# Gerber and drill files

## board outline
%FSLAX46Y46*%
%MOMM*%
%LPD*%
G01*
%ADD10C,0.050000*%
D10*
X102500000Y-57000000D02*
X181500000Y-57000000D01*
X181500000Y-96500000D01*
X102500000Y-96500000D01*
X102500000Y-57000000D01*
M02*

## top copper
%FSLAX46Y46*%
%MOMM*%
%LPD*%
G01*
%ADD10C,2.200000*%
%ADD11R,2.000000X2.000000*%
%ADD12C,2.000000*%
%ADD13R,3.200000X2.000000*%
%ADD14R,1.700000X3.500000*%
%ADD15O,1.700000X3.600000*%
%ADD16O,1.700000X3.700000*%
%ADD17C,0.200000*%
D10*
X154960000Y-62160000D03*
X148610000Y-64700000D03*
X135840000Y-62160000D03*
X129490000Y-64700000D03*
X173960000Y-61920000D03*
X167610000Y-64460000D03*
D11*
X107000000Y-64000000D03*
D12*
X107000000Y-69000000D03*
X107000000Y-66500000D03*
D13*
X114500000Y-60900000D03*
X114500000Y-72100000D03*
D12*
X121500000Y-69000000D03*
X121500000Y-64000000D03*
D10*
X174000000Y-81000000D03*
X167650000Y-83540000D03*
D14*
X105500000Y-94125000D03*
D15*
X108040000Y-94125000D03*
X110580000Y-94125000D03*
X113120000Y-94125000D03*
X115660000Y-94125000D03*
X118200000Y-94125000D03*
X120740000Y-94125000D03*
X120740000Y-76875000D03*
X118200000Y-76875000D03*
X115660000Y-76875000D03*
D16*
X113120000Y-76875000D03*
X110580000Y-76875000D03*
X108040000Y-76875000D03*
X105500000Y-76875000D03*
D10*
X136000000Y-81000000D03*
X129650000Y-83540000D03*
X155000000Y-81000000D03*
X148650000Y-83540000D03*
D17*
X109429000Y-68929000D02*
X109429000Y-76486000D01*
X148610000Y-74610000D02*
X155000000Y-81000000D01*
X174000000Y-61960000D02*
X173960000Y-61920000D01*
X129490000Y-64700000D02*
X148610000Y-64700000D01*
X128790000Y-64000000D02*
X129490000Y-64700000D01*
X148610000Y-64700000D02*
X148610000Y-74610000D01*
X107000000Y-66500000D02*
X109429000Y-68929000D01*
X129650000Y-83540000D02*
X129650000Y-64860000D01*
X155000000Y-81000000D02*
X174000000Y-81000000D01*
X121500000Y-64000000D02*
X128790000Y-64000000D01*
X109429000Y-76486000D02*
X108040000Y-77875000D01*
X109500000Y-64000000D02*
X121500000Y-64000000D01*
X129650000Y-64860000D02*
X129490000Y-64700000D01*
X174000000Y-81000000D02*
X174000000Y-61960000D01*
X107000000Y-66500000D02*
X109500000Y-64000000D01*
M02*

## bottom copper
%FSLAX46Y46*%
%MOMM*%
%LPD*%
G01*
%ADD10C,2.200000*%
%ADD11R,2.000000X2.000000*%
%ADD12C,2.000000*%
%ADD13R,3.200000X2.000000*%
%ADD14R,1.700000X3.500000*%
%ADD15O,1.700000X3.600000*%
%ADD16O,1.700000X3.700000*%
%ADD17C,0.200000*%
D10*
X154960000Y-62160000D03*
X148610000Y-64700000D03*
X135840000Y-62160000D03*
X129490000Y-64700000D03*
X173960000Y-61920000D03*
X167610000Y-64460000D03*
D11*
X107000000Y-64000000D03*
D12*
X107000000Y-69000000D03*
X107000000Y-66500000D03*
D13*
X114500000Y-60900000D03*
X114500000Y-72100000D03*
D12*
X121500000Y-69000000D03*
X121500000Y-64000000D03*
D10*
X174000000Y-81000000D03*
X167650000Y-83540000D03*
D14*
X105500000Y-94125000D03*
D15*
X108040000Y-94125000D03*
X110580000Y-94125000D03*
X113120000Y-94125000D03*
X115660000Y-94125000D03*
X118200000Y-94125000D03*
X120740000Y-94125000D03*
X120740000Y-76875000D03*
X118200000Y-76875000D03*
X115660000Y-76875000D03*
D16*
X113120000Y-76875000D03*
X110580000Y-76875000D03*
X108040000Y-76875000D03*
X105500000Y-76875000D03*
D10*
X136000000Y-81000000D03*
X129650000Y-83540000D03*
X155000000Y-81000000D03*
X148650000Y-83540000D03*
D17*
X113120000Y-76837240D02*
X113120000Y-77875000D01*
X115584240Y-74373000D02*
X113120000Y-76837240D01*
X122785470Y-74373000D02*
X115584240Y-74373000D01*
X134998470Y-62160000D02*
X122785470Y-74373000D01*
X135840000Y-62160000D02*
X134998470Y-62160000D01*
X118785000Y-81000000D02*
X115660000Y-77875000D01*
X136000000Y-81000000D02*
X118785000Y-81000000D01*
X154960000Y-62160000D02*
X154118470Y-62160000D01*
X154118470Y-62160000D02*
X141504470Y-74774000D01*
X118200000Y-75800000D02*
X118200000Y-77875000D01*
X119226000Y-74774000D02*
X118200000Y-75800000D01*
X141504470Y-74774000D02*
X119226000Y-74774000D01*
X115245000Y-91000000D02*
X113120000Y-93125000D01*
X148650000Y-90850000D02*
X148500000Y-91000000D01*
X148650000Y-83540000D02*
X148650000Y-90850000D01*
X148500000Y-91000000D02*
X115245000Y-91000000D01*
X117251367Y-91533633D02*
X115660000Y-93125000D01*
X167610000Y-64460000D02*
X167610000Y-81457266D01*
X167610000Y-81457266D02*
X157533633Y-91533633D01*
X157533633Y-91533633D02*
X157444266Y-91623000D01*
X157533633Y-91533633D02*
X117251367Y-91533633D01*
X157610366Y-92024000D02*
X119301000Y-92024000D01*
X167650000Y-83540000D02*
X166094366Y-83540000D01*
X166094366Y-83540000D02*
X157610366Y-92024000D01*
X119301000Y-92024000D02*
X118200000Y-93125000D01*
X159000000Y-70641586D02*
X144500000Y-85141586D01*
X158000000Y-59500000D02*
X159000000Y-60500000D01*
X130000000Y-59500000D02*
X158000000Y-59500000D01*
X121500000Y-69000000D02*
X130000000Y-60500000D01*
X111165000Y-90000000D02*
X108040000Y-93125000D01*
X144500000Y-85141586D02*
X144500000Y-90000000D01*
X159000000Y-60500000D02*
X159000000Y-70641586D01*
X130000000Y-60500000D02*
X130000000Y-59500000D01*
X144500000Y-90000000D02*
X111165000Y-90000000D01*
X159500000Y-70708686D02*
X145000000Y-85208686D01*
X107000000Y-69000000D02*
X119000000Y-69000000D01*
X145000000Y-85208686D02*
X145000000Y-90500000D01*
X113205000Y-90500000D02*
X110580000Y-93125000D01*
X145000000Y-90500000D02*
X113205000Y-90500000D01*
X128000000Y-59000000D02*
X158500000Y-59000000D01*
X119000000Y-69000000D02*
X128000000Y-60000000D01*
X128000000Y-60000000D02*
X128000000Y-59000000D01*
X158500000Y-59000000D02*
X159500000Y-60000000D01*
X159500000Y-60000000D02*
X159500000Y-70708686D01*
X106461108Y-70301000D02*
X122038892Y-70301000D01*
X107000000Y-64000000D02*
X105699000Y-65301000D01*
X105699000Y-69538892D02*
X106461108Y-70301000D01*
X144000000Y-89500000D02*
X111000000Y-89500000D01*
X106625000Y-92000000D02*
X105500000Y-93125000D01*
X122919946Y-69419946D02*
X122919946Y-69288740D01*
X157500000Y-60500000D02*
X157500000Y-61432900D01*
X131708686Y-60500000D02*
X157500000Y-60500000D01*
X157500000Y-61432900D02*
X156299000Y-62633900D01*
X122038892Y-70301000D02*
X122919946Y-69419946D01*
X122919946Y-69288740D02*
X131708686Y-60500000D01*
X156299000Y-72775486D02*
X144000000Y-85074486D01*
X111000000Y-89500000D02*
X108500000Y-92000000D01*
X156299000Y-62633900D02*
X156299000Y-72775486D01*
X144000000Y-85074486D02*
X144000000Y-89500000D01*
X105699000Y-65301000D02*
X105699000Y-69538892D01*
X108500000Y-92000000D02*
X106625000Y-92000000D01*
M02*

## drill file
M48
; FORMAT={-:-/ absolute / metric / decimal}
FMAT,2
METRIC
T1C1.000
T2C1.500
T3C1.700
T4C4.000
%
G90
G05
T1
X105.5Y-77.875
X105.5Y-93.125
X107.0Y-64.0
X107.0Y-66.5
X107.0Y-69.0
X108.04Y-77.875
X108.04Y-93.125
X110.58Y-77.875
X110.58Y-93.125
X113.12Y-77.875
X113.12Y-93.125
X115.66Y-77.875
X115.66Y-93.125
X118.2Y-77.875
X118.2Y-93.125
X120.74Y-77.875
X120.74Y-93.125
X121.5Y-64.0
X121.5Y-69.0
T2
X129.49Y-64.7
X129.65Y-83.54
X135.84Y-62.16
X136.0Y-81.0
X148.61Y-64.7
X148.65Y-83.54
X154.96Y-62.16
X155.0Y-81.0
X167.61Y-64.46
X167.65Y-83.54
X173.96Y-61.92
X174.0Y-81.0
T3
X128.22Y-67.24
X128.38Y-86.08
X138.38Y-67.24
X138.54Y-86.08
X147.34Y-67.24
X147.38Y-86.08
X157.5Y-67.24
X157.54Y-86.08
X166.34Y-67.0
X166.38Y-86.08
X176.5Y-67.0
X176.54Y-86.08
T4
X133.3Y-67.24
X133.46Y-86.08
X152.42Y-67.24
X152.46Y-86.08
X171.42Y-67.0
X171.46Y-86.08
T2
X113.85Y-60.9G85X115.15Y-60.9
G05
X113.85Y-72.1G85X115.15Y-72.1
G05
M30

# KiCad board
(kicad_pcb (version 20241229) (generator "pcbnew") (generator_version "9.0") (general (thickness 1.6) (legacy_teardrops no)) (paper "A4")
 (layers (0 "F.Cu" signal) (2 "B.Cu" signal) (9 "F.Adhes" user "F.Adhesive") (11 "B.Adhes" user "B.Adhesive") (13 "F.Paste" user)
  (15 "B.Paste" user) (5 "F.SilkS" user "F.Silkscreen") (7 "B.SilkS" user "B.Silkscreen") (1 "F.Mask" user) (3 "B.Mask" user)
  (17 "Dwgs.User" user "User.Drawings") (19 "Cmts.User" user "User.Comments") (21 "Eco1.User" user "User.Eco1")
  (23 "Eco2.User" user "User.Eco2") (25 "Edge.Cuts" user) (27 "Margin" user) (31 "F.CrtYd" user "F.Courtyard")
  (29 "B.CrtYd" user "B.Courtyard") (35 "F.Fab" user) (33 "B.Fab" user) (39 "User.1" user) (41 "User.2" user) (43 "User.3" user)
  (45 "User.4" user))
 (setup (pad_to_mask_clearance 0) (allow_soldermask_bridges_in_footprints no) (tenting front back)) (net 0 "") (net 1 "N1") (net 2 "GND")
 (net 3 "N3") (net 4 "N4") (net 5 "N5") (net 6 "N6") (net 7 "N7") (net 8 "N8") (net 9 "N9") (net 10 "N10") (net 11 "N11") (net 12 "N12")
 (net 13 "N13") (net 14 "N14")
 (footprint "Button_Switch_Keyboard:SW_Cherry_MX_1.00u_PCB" (layer "F.Cu") (at 154.96 62.16)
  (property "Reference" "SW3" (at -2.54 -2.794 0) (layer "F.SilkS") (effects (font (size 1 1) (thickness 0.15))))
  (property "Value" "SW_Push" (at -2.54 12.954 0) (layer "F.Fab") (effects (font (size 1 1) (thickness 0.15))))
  (pad "" np_thru_hole circle (at -7.62 5.08) (size 1.7 1.7) (drill 1.7) (layers "*.Cu" "*.Mask"))
  (pad "" np_thru_hole circle (at -2.54 5.08) (size 4 4) (drill 4) (layers "*.Cu" "*.Mask"))
  (pad "" np_thru_hole circle (at 2.54 5.08) (size 1.7 1.7) (drill 1.7) (layers "*.Cu" "*.Mask"))
  (pad "1" thru_hole circle (at 0 0) (size 2.2 2.2) (drill 1.5) (layers "*.Cu" "*.Mask") (remove_unused_layers no) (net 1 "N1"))
  (pad "2" thru_hole circle (at -6.35 2.54) (size 2.2 2.2) (drill 1.5) (layers "*.Cu" "*.Mask") (remove_unused_layers no) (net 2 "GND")))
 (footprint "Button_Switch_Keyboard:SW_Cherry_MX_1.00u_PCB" (layer "F.Cu") (at 135.84 62.16)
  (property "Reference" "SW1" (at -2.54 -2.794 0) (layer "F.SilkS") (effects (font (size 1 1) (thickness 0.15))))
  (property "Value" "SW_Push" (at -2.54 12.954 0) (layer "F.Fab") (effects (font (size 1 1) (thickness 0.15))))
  (pad "" np_thru_hole circle (at -7.62 5.08) (size 1.7 1.7) (drill 1.7) (layers "*.Cu" "*.Mask"))
  (pad "" np_thru_hole circle (at -2.54 5.08) (size 4 4) (drill 4) (layers "*.Cu" "*.Mask"))
  (pad "" np_thru_hole circle (at 2.54 5.08) (size 1.7 1.7) (drill 1.7) (layers "*.Cu" "*.Mask"))
  (pad "1" thru_hole circle (at 0 0) (size 2.2 2.2) (drill 1.5) (layers "*.Cu" "*.Mask") (remove_unused_layers no) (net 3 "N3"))
  (pad "2" thru_hole circle (at -6.35 2.54) (size 2.2 2.2) (drill 1.5) (layers "*.Cu" "*.Mask") (remove_unused_layers no) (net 2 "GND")))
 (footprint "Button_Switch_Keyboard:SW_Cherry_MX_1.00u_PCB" (layer "F.Cu") (at 173.96 61.92)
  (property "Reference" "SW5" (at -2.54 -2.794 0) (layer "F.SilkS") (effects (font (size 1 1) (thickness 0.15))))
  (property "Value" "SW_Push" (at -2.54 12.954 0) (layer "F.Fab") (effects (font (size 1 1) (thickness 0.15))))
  (pad "" np_thru_hole circle (at -7.62 5.08) (size 1.7 1.7) (drill 1.7) (layers "*.Cu" "*.Mask"))
  (pad "" np_thru_hole circle (at -2.54 5.08) (size 4 4) (drill 4) (layers "*.Cu" "*.Mask"))
  (pad "" np_thru_hole circle (at 2.54 5.08) (size 1.7 1.7) (drill 1.7) (layers "*.Cu" "*.Mask"))
  (pad "1" thru_hole circle (at 0 0) (size 2.2 2.2) (drill 1.5) (layers "*.Cu" "*.Mask") (remove_unused_layers no) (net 2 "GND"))
  (pad "2" thru_hole circle (at -6.35 2.54) (size 2.2 2.2) (drill 1.5) (layers "*.Cu" "*.Mask") (remove_unused_layers no) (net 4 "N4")))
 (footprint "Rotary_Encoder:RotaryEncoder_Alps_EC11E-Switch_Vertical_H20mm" (layer "F.Cu") (at 107 64)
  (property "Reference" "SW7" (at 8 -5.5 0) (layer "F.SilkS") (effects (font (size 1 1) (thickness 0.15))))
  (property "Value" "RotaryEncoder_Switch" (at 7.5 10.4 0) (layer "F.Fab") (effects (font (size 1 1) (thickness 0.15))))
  (pad "A" thru_hole rect (at 0 0) (size 2 2) (drill 1) (layers "*.Cu" "*.Mask") (remove_unused_layers no) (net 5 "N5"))
  (pad "B" thru_hole circle (at 0 5) (size 2 2) (drill 1) (layers "*.Cu" "*.Mask") (remove_unused_layers no) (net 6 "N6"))
  (pad "C" thru_hole circle (at 0 2.5) (size 2 2) (drill 1) (layers "*.Cu" "*.Mask") (remove_unused_layers no) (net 2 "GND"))
  (pad "MP" thru_hole rect (at 7.5 -3.1) (size 3.2 2) (drill oval 2.8 1.5) (layers "*.Cu" "*.Mask") (remove_unused_layers no))
  (pad "MP" thru_hole rect (at 7.5 8.1) (size 3.2 2) (drill oval 2.8 1.5) (layers "*.Cu" "*.Mask") (remove_unused_layers no))
  (pad "S1" thru_hole circle (at 14.5 5) (size 2 2) (drill 1) (layers "*.Cu" "*.Mask") (remove_unused_layers no) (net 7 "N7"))
  (pad "S2" thru_hole circle (at 14.5 0) (size 2 2) (drill 1) (layers "*.Cu" "*.Mask") (remove_unused_layers no) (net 2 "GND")))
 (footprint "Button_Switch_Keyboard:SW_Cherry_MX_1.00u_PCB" (layer "F.Cu") (at 174 81)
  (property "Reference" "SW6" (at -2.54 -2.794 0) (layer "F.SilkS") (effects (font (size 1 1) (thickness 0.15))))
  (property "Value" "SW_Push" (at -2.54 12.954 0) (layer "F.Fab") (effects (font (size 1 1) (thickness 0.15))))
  (pad "" np_thru_hole circle (at -7.62 5.08) (size 1.7 1.7) (drill 1.7) (layers "*.Cu" "*.Mask"))
  (pad "" np_thru_hole circle (at -2.54 5.08) (size 4 4) (drill 4) (layers "*.Cu" "*.Mask"))
  (pad "" np_thru_hole circle (at 2.54 5.08) (size 1.7 1.7) (drill 1.7) (layers "*.Cu" "*.Mask"))
  (pad "1" thru_hole circle (at 0 0) (size 2.2 2.2) (drill 1.5) (layers "*.Cu" "*.Mask") (remove_unused_layers no) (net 2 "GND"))
  (pad "2" thru_hole circle (at -6.35 2.54) (size 2.2 2.2) (drill 1.5) (layers "*.Cu" "*.Mask") (remove_unused_layers no) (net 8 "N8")))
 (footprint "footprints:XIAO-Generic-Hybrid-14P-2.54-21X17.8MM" (layer "F.Cu") (at 113.12 85.5 90)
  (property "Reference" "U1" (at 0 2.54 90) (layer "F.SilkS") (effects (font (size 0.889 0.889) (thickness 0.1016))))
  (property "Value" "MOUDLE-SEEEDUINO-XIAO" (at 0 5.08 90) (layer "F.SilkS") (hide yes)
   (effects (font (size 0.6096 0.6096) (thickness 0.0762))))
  (pad "1" thru_hole rect (at -7.625 -7.62 90) (size 3.5 1.7) (drill 1 (offset -1 0)) (layers "*.Cu" "*.Mask") (remove_unused_layers no)
   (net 5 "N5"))
  (pad "2" thru_hole oval (at -7.625 -5.08 90) (size 3.6 1.7) (drill 1 (offset -1 0)) (layers "*.Cu" "*.Mask") (remove_unused_layers no)
   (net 7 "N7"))
  (pad "3" thru_hole oval (at -7.625 -2.54 90) (size 3.6 1.7) (drill 1 (offset -1 0)) (layers "*.Cu" "*.Mask") (remove_unused_layers no)
   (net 6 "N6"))
  (pad "4" thru_hole oval (at -7.625 0 90) (size 3.6 1.7) (drill 1 (offset -1 0)) (layers "*.Cu" "*.Mask") (remove_unused_layers no)
   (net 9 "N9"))
  (pad "5" thru_hole oval (at -7.625 2.54 90) (size 3.6 1.7) (drill 1 (offset -1 0)) (layers "*.Cu" "*.Mask") (remove_unused_layers no)
   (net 4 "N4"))
  (pad "6" thru_hole oval (at -7.625 5.08 270) (size 3.6 1.7) (drill 1 (offset 1 0)) (layers "*.Cu" "*.Mask") (remove_unused_layers no)
   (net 8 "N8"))
  (pad "7" thru_hole oval (at -7.625 7.62 90) (size 3.6 1.7) (drill 1 (offset -1 0)) (layers "*.Cu" "*.Mask") (remove_unused_layers no)
   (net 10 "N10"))
  (pad "8" thru_hole oval (at 7.625 7.62 90) (size 3.6 1.7) (drill 1 (offset 1 0)) (layers "*.Cu" "*.Mask") (remove_unused_layers no)
   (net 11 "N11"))
  (pad "9" thru_hole oval (at 7.625 5.08 90) (size 3.6 1.7) (drill 1 (offset 1 0)) (layers "*.Cu" "*.Mask") (remove_unused_layers no)
   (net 1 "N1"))
  (pad "10" thru_hole oval (at 7.625 2.54 90) (size 3.6 1.7) (drill 1 (offset 1 0)) (layers "*.Cu" "*.Mask") (remove_unused_layers no)
   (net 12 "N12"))
  (pad "11" thru_hole oval (at 7.625 0 90) (size 3.7 1.7) (drill 1 (offset 1 0)) (layers "*.Cu" "*.Mask") (remove_unused_layers no)
   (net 3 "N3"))
  (pad "12" thru_hole oval (at 7.625 -2.54 90) (size 3.7 1.7) (drill 1 (offset 1 0)) (layers "*.Cu" "*.Mask") (remove_unused_layers no)
   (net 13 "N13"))
  (pad "13" thru_hole oval (at 7.625 -5.08 90) (size 3.7 1.7) (drill 1 (offset 1 0)) (layers "*.Cu" "*.Mask") (remove_unused_layers no)
   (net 2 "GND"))
  (pad "14" thru_hole oval (at 7.625 -7.62 90) (size 3.7 1.7) (drill 1 (offset 1 0)) (layers "*.Cu" "*.Mask") (remove_unused_layers no)
   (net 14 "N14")))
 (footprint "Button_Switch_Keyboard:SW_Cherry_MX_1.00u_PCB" (layer "F.Cu") (at 136 81)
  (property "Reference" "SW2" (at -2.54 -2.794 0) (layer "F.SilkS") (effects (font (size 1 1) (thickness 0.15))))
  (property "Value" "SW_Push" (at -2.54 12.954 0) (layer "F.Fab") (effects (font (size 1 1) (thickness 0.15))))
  (pad "" np_thru_hole circle (at -7.62 5.08) (size 1.7 1.7) (drill 1.7) (layers "*.Cu" "*.Mask"))
  (pad "" np_thru_hole circle (at -2.54 5.08) (size 4 4) (drill 4) (layers "*.Cu" "*.Mask"))
  (pad "" np_thru_hole circle (at 2.54 5.08) (size 1.7 1.7) (drill 1.7) (layers "*.Cu" "*.Mask"))
  (pad "1" thru_hole circle (at 0 0) (size 2.2 2.2) (drill 1.5) (layers "*.Cu" "*.Mask") (remove_unused_layers no) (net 12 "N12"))
  (pad "2" thru_hole circle (at -6.35 2.54) (size 2.2 2.2) (drill 1.5) (layers "*.Cu" "*.Mask") (remove_unused_layers no) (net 2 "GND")))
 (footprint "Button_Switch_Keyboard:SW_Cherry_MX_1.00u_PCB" (layer "F.Cu") (at 155 81)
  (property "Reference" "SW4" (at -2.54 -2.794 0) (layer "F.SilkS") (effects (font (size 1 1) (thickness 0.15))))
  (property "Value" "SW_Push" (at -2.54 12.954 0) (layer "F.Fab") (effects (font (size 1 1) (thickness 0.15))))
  (pad "" np_thru_hole circle (at -7.62 5.08) (size 1.7 1.7) (drill 1.7) (layers "*.Cu" "*.Mask"))
  (pad "" np_thru_hole circle (at -2.54 5.08) (size 4 4) (drill 4) (layers "*.Cu" "*.Mask"))
  (pad "" np_thru_hole circle (at 2.54 5.08) (size 1.7 1.7) (drill 1.7) (layers "*.Cu" "*.Mask"))
  (pad "1" thru_hole circle (at 0 0) (size 2.2 2.2) (drill 1.5) (layers "*.Cu" "*.Mask") (remove_unused_layers no) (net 2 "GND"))
  (pad "2" thru_hole circle (at -6.35 2.54) (size 2.2 2.2) (drill 1.5) (layers "*.Cu" "*.Mask") (remove_unused_layers no) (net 9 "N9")))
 (gr_rect (start 102.5 57) (end 181.5 96.5) (stroke (width 0.05) (type default)) (fill no) (layer "Edge.Cuts"))
 (segment (start 113.12 76.83724) (end 113.12 77.875) (width 0.2) (layer "B.Cu") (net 3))
 (segment (start 115.58424 74.373) (end 113.12 76.83724) (width 0.2) (layer "B.Cu") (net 3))
 (segment (start 122.78547 74.373) (end 115.58424 74.373) (width 0.2) (layer "B.Cu") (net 3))
 (segment (start 134.99847 62.16) (end 122.78547 74.373) (width 0.2) (layer "B.Cu") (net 3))
 (segment (start 135.84 62.16) (end 134.99847 62.16) (width 0.2) (layer "B.Cu") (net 3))
 (segment (start 109.429 68.929) (end 109.429 76.486) (width 0.2) (layer "F.Cu") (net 2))
 (segment (start 148.61 74.61) (end 155 81) (width 0.2) (layer "F.Cu") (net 2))
 (segment (start 174 61.96) (end 173.96 61.92) (width 0.2) (layer "F.Cu") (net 2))
 (segment (start 129.49 64.7) (end 148.61 64.7) (width 0.2) (layer "F.Cu") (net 2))
 (segment (start 128.79 64) (end 129.49 64.7) (width 0.2) (layer "F.Cu") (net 2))
 (segment (start 148.61 64.7) (end 148.61 74.61) (width 0.2) (layer "F.Cu") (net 2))
 (segment (start 107 66.5) (end 109.429 68.929) (width 0.2) (layer "F.Cu") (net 2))
 (segment (start 129.65 83.54) (end 129.65 64.86) (width 0.2) (layer "F.Cu") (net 2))
 (segment (start 155 81) (end 174 81) (width 0.2) (layer "F.Cu") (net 2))
 (segment (start 121.5 64) (end 128.79 64) (width 0.2) (layer "F.Cu") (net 2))
 (segment (start 109.429 76.486) (end 108.04 77.875) (width 0.2) (layer "F.Cu") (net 2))
 (segment (start 109.5 64) (end 121.5 64) (width 0.2) (layer "F.Cu") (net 2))
 (segment (start 129.65 64.86) (end 129.49 64.7) (width 0.2) (layer "F.Cu") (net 2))
 (segment (start 174 81) (end 174 61.96) (width 0.2) (layer "F.Cu") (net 2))
 (segment (start 107 66.5) (end 109.5 64) (width 0.2) (layer "F.Cu") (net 2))
 (segment (start 118.785 81) (end 115.66 77.875) (width 0.2) (layer "B.Cu") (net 12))
 (segment (start 136 81) (end 118.785 81) (width 0.2) (layer "B.Cu") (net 12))
 (segment (start 154.96 62.16) (end 154.11847 62.16) (width 0.2) (layer "B.Cu") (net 1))
 (segment (start 154.11847 62.16) (end 141.50447 74.774) (width 0.2) (layer "B.Cu") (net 1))
 (segment (start 118.2 75.8) (end 118.2 77.875) (width 0.2) (layer "B.Cu") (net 1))
 (segment (start 119.226 74.774) (end 118.2 75.8) (width 0.2) (layer "B.Cu") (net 1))
 (segment (start 141.50447 74.774) (end 119.226 74.774) (width 0.2) (layer "B.Cu") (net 1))
 (segment (start 115.245 91) (end 113.12 93.125) (width 0.2) (layer "B.Cu") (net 9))
 (segment (start 148.65 90.85) (end 148.5 91) (width 0.2) (layer "B.Cu") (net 9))
 (segment (start 148.65 83.54) (end 148.65 90.85) (width 0.2) (layer "B.Cu") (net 9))
 (segment (start 148.5 91) (end 115.245 91) (width 0.2) (layer "B.Cu") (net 9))
 (segment (start 117.251367 91.533633) (end 115.66 93.125) (width 0.2) (layer "B.Cu") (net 4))
 (segment (start 167.61 64.46) (end 167.61 81.457266) (width 0.2) (layer "B.Cu") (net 4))
 (segment (start 167.61 81.457266) (end 157.533633 91.533633) (width 0.2) (layer "B.Cu") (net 4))
 (segment (start 157.533633 91.533633) (end 157.444266 91.623) (width 0.2) (layer "B.Cu") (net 4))
 (segment (start 157.533633 91.533633) (end 117.251367 91.533633) (width 0.2) (layer "B.Cu") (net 4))
 (segment (start 157.610366 92.024) (end 119.301 92.024) (width 0.2) (layer "B.Cu") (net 8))
 (segment (start 167.65 83.54) (end 166.094366 83.54) (width 0.2) (layer "B.Cu") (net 8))
 (segment (start 166.094366 83.54) (end 157.610366 92.024) (width 0.2) (layer "B.Cu") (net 8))
 (segment (start 119.301 92.024) (end 118.2 93.125) (width 0.2) (layer "B.Cu") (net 8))
 (segment (start 159 70.641586) (end 144.5 85.141586) (width 0.2) (layer "B.Cu") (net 7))
 (segment (start 158 59.5) (end 159 60.5) (width 0.2) (layer "B.Cu") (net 7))
 (segment (start 130 59.5) (end 158 59.5) (width 0.2) (layer "B.Cu") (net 7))
 (segment (start 121.5 69) (end 130 60.5) (width 0.2) (layer "B.Cu") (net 7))
 (segment (start 111.165 90) (end 108.04 93.125) (width 0.2) (layer "B.Cu") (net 7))
 (segment (start 144.5 85.141586) (end 144.5 90) (width 0.2) (layer "B.Cu") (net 7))
 (segment (start 159 60.5) (end 159 70.641586) (width 0.2) (layer "B.Cu") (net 7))
 (segment (start 130 60.5) (end 130 59.5) (width 0.2) (layer "B.Cu") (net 7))
 (segment (start 144.5 90) (end 111.165 90) (width 0.2) (layer "B.Cu") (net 7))
 (segment (start 159.5 70.708686) (end 145 85.208686) (width 0.2) (layer "B.Cu") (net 6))
 (segment (start 107 69) (end 119 69) (width 0.2) (layer "B.Cu") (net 6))
 (segment (start 145 85.208686) (end 145 90.5) (width 0.2) (layer "B.Cu") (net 6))
 (segment (start 113.205 90.5) (end 110.58 93.125) (width 0.2) (layer "B.Cu") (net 6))
 (segment (start 145 90.5) (end 113.205 90.5) (width 0.2) (layer "B.Cu") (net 6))
 (segment (start 128 59) (end 158.5 59) (width 0.2) (layer "B.Cu") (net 6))
 (segment (start 119 69) (end 128 60) (width 0.2) (layer "B.Cu") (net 6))
 (segment (start 128 60) (end 128 59) (width 0.2) (layer "B.Cu") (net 6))
 (segment (start 158.5 59) (end 159.5 60) (width 0.2) (layer "B.Cu") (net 6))
 (segment (start 159.5 60) (end 159.5 70.708686) (width 0.2) (layer "B.Cu") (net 6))
 (segment (start 106.461108 70.301) (end 122.038892 70.301) (width 0.2) (layer "B.Cu") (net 5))
 (segment (start 107 64) (end 105.699 65.301) (width 0.2) (layer "B.Cu") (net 5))
 (segment (start 105.699 69.538892) (end 106.461108 70.301) (width 0.2) (layer "B.Cu") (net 5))
 (segment (start 144 89.5) (end 111 89.5) (width 0.2) (layer "B.Cu") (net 5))
 (segment (start 106.625 92) (end 105.5 93.125) (width 0.2) (layer "B.Cu") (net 5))
 (segment (start 122.919946 69.419946) (end 122.919946 69.28874) (width 0.2) (layer "B.Cu") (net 5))
 (segment (start 157.5 60.5) (end 157.5 61.4329) (width 0.2) (layer "B.Cu") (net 5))
 (segment (start 131.708686 60.5) (end 157.5 60.5) (width 0.2) (layer "B.Cu") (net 5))
 (segment (start 157.5 61.4329) (end 156.299 62.6339) (width 0.2) (layer "B.Cu") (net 5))
 (segment (start 122.038892 70.301) (end 122.919946 69.419946) (width 0.2) (layer "B.Cu") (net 5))
 (segment (start 122.919946 69.28874) (end 131.708686 60.5) (width 0.2) (layer "B.Cu") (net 5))
 (segment (start 156.299 72.775486) (end 144 85.074486) (width 0.2) (layer "B.Cu") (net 5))
 (segment (start 111 89.5) (end 108.5 92) (width 0.2) (layer "B.Cu") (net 5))
 (segment (start 156.299 62.6339) (end 156.299 72.775486) (width 0.2) (layer "B.Cu") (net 5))
 (segment (start 144 85.074486) (end 144 89.5) (width 0.2) (layer "B.Cu") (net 5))
 (segment (start 105.699 65.301) (end 105.699 69.538892) (width 0.2) (layer "B.Cu") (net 5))
 (segment (start 108.5 92) (end 106.625 92) (width 0.2) (layer "B.Cu") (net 5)))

